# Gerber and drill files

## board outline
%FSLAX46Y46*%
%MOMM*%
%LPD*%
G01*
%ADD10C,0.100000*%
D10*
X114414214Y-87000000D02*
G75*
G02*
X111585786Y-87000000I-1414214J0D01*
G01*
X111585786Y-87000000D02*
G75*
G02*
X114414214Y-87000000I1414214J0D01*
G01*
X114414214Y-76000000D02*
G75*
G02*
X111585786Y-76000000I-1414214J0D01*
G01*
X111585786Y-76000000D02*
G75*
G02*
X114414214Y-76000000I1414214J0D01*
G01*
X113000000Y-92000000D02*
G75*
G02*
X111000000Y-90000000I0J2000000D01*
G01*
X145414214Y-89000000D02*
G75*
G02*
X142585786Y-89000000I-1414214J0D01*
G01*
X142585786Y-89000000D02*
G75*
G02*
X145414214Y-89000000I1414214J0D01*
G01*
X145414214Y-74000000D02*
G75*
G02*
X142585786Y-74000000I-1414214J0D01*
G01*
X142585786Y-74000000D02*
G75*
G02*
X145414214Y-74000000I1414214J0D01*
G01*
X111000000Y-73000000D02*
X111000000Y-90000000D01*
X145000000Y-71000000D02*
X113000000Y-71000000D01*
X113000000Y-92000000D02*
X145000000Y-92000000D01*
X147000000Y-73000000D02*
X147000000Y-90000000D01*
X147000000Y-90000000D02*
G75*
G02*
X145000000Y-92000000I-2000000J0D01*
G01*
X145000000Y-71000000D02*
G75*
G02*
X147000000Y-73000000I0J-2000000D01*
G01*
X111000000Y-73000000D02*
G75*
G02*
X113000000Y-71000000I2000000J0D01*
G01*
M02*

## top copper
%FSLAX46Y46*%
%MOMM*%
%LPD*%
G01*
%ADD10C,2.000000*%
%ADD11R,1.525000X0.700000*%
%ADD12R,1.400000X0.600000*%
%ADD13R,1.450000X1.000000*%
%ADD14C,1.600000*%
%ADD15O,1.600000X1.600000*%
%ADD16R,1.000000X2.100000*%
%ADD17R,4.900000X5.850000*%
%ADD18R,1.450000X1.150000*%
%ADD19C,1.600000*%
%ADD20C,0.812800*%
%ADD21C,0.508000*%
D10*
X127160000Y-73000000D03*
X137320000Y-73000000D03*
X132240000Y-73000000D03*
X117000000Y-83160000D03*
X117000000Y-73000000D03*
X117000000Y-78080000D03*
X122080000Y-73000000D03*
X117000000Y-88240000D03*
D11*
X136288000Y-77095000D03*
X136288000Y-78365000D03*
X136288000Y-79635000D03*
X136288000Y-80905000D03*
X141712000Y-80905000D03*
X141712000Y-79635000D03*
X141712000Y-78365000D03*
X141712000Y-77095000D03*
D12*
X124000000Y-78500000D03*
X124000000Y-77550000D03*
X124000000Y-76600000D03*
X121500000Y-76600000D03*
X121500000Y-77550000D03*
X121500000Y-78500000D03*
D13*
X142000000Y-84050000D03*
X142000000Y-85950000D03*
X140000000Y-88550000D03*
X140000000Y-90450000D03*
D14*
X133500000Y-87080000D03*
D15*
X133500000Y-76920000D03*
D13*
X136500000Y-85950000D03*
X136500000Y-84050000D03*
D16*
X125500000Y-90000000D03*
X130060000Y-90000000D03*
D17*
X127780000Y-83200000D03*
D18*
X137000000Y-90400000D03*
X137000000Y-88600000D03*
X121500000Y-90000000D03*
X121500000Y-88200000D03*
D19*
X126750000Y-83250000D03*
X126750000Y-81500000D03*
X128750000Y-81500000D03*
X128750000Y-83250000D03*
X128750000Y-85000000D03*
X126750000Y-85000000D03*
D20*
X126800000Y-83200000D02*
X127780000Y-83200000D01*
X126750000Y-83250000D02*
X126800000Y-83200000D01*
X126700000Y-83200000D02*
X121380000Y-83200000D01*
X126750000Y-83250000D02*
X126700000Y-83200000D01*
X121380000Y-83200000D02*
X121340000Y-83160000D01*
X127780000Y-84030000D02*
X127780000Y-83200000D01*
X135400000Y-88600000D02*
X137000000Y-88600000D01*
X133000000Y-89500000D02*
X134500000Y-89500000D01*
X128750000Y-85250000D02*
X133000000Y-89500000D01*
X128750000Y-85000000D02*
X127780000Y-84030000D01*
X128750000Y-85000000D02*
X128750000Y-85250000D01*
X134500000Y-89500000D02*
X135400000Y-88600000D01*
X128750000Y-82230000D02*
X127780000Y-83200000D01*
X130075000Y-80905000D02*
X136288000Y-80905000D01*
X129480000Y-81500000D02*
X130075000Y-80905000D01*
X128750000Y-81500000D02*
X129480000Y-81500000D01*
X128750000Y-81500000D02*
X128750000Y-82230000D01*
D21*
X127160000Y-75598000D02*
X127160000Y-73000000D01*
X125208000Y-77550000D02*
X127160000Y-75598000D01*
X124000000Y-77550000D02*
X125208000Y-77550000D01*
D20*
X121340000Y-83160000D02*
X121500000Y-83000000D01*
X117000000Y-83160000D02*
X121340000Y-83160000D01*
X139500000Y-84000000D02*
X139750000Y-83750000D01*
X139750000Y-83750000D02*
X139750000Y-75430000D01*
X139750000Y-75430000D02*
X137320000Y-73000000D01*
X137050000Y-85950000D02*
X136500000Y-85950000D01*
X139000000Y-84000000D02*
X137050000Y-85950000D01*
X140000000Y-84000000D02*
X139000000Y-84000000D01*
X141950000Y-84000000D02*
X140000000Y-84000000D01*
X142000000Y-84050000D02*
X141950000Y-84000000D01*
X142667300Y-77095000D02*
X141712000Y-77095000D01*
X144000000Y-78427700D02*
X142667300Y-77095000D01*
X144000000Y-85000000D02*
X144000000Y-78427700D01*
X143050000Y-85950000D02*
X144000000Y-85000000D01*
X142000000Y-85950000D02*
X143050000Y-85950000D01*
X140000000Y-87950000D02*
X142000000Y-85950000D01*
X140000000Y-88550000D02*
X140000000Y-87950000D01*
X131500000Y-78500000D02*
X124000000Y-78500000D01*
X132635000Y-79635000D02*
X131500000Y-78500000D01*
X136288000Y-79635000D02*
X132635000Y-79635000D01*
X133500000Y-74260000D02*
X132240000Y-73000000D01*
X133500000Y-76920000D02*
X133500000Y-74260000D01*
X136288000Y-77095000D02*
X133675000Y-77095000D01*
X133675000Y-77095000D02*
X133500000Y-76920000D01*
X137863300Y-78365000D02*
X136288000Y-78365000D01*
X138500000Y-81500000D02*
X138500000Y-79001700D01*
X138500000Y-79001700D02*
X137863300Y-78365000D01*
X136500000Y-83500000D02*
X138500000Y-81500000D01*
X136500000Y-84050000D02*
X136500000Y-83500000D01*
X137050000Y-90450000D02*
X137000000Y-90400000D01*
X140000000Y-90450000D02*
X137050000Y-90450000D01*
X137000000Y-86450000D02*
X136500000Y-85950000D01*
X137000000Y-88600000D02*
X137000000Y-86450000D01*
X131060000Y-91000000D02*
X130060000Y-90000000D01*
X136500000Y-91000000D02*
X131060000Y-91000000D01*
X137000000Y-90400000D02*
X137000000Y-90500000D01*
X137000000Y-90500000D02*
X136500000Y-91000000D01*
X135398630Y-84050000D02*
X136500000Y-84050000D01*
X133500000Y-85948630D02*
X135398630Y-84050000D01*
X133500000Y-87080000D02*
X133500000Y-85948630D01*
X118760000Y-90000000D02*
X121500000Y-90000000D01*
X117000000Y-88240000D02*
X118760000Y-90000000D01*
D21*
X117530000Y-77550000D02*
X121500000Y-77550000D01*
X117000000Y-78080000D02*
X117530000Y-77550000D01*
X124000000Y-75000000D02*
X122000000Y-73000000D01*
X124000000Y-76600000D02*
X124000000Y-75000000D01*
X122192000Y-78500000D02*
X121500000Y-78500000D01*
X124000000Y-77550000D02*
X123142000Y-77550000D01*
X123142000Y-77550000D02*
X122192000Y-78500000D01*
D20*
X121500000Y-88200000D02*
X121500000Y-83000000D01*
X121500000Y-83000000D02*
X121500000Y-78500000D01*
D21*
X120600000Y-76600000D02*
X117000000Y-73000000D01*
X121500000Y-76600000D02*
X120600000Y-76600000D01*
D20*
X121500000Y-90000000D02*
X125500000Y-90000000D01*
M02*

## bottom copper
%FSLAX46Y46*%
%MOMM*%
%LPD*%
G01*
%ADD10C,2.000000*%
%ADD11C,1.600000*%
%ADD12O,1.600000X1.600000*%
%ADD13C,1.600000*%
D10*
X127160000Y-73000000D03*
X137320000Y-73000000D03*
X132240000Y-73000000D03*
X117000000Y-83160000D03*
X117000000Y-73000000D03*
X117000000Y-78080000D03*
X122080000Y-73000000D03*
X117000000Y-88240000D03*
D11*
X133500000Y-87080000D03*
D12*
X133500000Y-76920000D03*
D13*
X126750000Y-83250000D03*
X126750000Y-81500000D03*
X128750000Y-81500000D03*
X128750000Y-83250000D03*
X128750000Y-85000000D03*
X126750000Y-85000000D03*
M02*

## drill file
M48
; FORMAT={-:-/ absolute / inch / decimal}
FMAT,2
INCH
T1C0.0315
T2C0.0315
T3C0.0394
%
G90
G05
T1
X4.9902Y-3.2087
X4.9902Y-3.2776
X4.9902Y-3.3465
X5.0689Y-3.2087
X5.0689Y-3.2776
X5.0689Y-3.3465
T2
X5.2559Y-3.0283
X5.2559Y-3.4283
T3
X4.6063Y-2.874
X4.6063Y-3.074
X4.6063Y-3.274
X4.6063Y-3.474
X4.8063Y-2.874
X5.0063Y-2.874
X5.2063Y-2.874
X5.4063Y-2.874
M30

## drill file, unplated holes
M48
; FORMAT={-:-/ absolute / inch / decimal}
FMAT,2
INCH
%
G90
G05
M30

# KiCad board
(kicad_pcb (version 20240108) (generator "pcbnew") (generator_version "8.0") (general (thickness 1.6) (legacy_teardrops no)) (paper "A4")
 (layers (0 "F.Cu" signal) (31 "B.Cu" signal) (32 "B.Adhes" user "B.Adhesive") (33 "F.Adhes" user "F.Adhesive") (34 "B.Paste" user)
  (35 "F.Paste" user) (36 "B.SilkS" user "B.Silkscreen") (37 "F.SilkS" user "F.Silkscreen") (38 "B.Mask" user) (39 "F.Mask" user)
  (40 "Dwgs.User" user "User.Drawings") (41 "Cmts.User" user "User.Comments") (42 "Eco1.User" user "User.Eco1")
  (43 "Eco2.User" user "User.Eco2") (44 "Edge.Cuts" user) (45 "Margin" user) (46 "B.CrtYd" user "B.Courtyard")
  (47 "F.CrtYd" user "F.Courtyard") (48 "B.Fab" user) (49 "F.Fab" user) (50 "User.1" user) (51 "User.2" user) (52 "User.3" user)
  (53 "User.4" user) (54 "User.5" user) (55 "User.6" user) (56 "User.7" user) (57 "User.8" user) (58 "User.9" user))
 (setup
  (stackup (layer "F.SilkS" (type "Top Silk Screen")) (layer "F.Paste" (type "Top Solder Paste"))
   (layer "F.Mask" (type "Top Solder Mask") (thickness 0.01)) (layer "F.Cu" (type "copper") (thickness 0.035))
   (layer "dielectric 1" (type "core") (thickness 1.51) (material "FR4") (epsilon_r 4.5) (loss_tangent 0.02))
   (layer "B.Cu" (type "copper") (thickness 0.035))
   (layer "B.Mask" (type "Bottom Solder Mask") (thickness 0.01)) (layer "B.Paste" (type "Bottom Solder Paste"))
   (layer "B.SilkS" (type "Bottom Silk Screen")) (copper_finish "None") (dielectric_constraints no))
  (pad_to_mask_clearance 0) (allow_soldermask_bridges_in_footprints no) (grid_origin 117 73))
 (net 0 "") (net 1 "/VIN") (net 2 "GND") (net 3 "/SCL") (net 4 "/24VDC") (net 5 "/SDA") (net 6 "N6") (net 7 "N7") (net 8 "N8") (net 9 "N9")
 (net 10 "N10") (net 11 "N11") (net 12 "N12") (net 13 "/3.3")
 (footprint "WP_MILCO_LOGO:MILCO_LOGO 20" (layer "F.Cu") (at 113.5 81.4 90)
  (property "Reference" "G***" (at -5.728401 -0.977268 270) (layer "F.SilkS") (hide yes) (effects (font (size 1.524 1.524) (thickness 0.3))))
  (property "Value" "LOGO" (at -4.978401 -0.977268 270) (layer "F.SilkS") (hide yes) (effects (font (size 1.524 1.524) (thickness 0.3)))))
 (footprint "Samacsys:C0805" (layer "F.Cu") (at 121.5 89.1 90)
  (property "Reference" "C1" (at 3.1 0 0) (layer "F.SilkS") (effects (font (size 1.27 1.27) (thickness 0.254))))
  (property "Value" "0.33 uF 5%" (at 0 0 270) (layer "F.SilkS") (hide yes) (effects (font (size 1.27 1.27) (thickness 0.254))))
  (pad "1" smd rect (at -0.9 0 90) (size 1.15 1.45) (layers "F.Cu" "F.Paste" "F.Mask") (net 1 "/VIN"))
  (pad "2" smd rect (at 0.9 0 90) (size 1.15 1.45) (layers "F.Cu" "F.Paste" "F.Mask") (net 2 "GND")))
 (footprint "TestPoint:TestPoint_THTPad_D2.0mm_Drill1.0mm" (layer "F.Cu") (at 127.16 73)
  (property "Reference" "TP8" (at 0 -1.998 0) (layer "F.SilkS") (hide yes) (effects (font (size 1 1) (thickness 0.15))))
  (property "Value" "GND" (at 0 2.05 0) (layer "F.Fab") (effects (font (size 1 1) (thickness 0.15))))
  (pad "1" thru_hole circle (at 0 0) (size 2 2) (drill 1) (layers "*.Cu" "*.Mask") (remove_unused_layers no) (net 2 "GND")))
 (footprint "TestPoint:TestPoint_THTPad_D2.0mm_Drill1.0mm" (layer "F.Cu") (at 117 78.08)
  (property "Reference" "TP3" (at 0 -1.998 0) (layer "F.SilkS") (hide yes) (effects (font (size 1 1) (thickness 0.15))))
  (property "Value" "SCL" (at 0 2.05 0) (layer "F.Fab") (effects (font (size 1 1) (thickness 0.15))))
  (pad "1" thru_hole circle (at 0 0) (size 2 2) (drill 1) (layers "*.Cu" "*.Mask") (remove_unused_layers no) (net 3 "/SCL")))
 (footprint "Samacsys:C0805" (layer "F.Cu") (at 137 89.5 90)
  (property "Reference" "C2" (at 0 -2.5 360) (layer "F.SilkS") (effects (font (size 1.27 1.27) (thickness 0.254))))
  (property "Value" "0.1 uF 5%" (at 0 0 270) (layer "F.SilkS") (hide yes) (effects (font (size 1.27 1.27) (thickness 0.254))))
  (pad "1" smd rect (at -0.9 0 90) (size 1.15 1.45) (layers "F.Cu" "F.Paste" "F.Mask") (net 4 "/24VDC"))
  (pad "2" smd rect (at 0.9 0 90) (size 1.15 1.45) (layers "F.Cu" "F.Paste" "F.Mask") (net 2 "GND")))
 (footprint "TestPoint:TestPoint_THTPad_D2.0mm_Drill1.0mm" (layer "F.Cu") (at 117 73)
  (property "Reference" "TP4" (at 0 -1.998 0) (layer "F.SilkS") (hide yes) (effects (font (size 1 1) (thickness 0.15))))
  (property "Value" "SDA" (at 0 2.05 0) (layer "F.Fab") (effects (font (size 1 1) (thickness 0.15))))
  (pad "1" thru_hole circle (at 0 0) (size 2 2) (drill 1) (layers "*.Cu" "*.Mask") (remove_unused_layers no) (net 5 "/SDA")))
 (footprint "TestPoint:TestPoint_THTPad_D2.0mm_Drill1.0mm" (layer "F.Cu") (at 117 83.16)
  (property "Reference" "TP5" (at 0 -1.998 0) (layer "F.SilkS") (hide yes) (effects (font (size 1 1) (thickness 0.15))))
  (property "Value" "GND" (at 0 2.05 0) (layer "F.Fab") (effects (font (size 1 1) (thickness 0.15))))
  (pad "1" thru_hole circle (at 0 0) (size 2 2) (drill 1) (layers "*.Cu" "*.Mask") (remove_unused_layers no) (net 2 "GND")))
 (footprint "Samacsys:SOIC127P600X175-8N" (layer "F.Cu") (at 139 79)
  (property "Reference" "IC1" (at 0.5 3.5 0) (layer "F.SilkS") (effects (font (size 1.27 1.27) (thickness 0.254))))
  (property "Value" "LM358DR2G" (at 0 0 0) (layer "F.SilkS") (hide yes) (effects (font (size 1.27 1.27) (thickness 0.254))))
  (pad "1" smd rect (at -2.712 -1.905 90) (size 0.7 1.525) (layers "F.Cu" "F.Paste" "F.Mask") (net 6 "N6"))
  (pad "2" smd rect (at -2.712 -0.635 90) (size 0.7 1.525) (layers "F.Cu" "F.Paste" "F.Mask") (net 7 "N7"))
  (pad "3" smd rect (at -2.712 0.635 90) (size 0.7 1.525) (layers "F.Cu" "F.Paste" "F.Mask") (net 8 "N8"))
  (pad "4" smd rect (at -2.712 1.905 90) (size 0.7 1.525) (layers "F.Cu" "F.Paste" "F.Mask") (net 2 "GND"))
  (pad "5" smd rect (at 2.712 1.905 90) (size 0.7 1.525) (layers "F.Cu" "F.Paste" "F.Mask") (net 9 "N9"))
  (pad "6" smd rect (at 2.712 0.635 90) (size 0.7 1.525) (layers "F.Cu" "F.Paste" "F.Mask") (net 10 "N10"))
  (pad "7" smd rect (at 2.712 -0.635 90) (size 0.7 1.525) (layers "F.Cu" "F.Paste" "F.Mask") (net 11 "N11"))
  (pad "8" smd rect (at 2.712 -1.905 90) (size 0.7 1.525) (layers "F.Cu" "F.Paste" "F.Mask") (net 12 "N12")))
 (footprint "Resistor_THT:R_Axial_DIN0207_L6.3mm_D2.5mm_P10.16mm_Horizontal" (layer "F.Cu") (at 133.5 87.08 90)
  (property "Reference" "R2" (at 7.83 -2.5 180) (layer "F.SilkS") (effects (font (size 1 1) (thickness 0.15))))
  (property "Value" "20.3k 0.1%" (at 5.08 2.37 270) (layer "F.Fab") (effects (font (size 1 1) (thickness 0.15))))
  (pad "1" thru_hole circle (at 0 0 90) (size 1.6 1.6) (drill 0.8) (layers "*.Cu" "*.Mask") (remove_unused_layers no) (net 7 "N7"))
  (pad "2" thru_hole oval (at 10.16 0 90) (size 1.6 1.6) (drill 0.8) (layers "*.Cu" "*.Mask") (remove_unused_layers no) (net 6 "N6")))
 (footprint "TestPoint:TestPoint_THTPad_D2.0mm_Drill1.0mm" (layer "F.Cu") (at 132.24 73)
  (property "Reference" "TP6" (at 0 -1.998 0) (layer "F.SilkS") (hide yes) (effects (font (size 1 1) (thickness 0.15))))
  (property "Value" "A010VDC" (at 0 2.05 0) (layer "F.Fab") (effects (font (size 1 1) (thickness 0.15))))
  (pad "1" thru_hole circle (at 0 0) (size 2 2) (drill 1) (layers "*.Cu" "*.Mask") (remove_unused_layers no) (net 6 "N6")))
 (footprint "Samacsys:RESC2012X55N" (layer "F.Cu") (at 136.5 85 90)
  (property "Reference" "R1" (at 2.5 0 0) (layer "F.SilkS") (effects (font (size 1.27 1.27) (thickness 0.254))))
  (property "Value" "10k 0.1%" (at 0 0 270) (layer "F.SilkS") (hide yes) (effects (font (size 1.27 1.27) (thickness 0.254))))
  (pad "1" smd rect (at -0.95 0 90) (size 1 1.45) (layers "F.Cu" "F.Paste" "F.Mask") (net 2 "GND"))
  (pad "2" smd rect (at 0.95 0 90) (size 1 1.45) (layers "F.Cu" "F.Paste" "F.Mask") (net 7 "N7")))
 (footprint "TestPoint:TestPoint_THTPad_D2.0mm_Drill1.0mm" (layer "F.Cu") (at 137.32 73)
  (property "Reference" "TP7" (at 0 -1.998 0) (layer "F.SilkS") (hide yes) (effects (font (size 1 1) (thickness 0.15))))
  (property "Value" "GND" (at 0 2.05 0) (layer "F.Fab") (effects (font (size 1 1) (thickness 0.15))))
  (pad "1" thru_hole circle (at 0 0) (size 2 2) (drill 1) (layers "*.Cu" "*.Mask") (remove_unused_layers no) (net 2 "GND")))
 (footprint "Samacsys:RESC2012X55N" (layer "F.Cu") (at 140 89.5 -90)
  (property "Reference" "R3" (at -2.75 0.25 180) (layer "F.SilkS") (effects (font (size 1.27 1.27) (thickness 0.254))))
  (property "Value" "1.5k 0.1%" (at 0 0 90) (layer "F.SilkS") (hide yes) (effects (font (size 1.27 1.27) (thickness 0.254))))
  (pad "1" smd rect (at -0.95 0 270) (size 1 1.45) (layers "F.Cu" "F.Paste" "F.Mask") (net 12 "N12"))
  (pad "2" smd rect (at 0.95 0 270) (size 1 1.45) (layers "F.Cu" "F.Paste" "F.Mask") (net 4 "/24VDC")))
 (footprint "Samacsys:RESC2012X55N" (layer "F.Cu") (at 142 85 -90)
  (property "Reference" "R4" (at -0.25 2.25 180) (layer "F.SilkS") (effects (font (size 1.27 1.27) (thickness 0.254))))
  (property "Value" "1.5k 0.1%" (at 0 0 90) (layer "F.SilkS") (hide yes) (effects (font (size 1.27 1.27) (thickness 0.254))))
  (pad "1" smd rect (at -0.95 0 270) (size 1 1.45) (layers "F.Cu" "F.Paste" "F.Mask") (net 2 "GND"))
  (pad "2" smd rect (at 0.95 0 270) (size 1 1.45) (layers "F.Cu" "F.Paste" "F.Mask") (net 12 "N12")))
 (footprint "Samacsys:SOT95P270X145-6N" (layer "F.Cu") (at 122.75 77.55 180)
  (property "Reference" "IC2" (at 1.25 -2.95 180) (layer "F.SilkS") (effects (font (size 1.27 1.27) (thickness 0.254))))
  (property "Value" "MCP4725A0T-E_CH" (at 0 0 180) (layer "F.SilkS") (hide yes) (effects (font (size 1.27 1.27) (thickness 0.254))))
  (pad "1" smd rect (at -1.25 -0.95 270) (size 0.6 1.4) (layers "F.Cu" "F.Paste" "F.Mask") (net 8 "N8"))
  (pad "2" smd rect (at -1.25 0 270) (size 0.6 1.4) (layers "F.Cu" "F.Paste" "F.Mask") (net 2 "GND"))
  (pad "3" smd rect (at -1.25 0.95 270) (size 0.6 1.4) (layers "F.Cu" "F.Paste" "F.Mask") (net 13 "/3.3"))
  (pad "4" smd rect (at 1.25 0.95 270) (size 0.6 1.4) (layers "F.Cu" "F.Paste" "F.Mask") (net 5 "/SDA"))
  (pad "5" smd rect (at 1.25 0 270) (size 0.6 1.4) (layers "F.Cu" "F.Paste" "F.Mask") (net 3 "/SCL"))
  (pad "6" smd rect (at 1.25 -0.95 270) (size 0.6 1.4) (layers "F.Cu" "F.Paste" "F.Mask") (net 2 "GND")))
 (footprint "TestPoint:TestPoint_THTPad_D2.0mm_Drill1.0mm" (layer "F.Cu") (at 117 88.24)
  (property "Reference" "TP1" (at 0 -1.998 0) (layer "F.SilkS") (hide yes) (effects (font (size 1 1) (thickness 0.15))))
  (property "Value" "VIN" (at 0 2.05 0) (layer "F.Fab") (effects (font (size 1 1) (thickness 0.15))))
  (pad "1" thru_hole circle (at 0 0) (size 2 2) (drill 1) (layers "*.Cu" "*.Mask") (remove_unused_layers no) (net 1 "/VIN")))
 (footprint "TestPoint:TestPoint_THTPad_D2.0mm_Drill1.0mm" (layer "F.Cu") (at 122.08 73)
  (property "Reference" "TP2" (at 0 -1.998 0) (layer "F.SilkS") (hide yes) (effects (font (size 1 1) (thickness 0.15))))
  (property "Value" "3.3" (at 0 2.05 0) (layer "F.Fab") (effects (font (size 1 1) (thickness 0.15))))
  (pad "1" thru_hole circle (at 0 0) (size 2 2) (drill 1) (layers "*.Cu" "*.Mask") (remove_unused_layers no) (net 13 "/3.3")))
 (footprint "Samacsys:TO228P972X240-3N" (layer "F.Cu") (at 127.78 85.65 90)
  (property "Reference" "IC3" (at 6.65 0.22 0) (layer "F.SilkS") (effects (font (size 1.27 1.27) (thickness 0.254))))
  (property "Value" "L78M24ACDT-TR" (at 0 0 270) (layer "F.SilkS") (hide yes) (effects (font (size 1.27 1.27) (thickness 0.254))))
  (pad "1" smd rect (at -4.35 -2.28 180) (size 1 2.1) (layers "F.Cu" "F.Paste" "F.Mask") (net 1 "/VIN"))
  (pad "3" smd rect (at -4.35 2.28 180) (size 1 2.1) (layers "F.Cu" "F.Paste" "F.Mask") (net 4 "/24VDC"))
  (pad "4" smd rect (at 2.45 0 180) (size 4.9 5.85) (layers "F.Cu" "F.Paste" "F.Mask") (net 2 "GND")))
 (gr_arc (start 111 73) (mid 111.585786 71.585786) (end 113 71) (stroke (width 0.1) (type default)) (layer "Edge.Cuts"))
 (gr_circle (center 144 89) (end 145 90) (stroke (width 0.1) (type default)) (fill none) (layer "Edge.Cuts"))
 (gr_arc (start 145 71) (mid 146.414214 71.585786) (end 147 73) (stroke (width 0.1) (type default)) (layer "Edge.Cuts"))
 (gr_circle (center 113 87) (end 112 86) (stroke (width 0.1) (type default)) (fill none) (layer "Edge.Cuts"))
 (gr_line (start 145 71) (end 113 71) (stroke (width 0.1) (type default)) (layer "Edge.Cuts"))
 (gr_circle (center 113 76) (end 112 75) (stroke (width 0.1) (type default)) (fill none) (layer "Edge.Cuts"))
 (gr_line (start 147 73) (end 147 90) (stroke (width 0.1) (type default)) (layer "Edge.Cuts"))
 (gr_arc (start 113 92) (mid 111.585786 91.414214) (end 111 90) (stroke (width 0.1) (type default)) (layer "Edge.Cuts"))
 (gr_circle (center 144 74) (end 145 73) (stroke (width 0.1) (type default)) (fill none) (layer "Edge.Cuts"))
 (gr_line (start 113 92) (end 145 92) (stroke (width 0.1) (type default)) (layer "Edge.Cuts"))
 (gr_arc (start 147 90) (mid 146.414214 91.414214) (end 145 92) (stroke (width 0.1) (type default)) (layer "Edge.Cuts"))
 (gr_line (start 111 73) (end 111 90) (stroke (width 0.1) (type default)) (layer "Edge.Cuts"))
 (segment (start 118.76 90) (end 121.5 90) (width 0.8128) (layer "F.Cu") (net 1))
 (segment (start 121.5 90) (end 125.5 90) (width 0.8128) (layer "F.Cu") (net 1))
 (segment (start 117 88.24) (end 118.76 90) (width 0.8128) (layer "F.Cu") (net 1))
 (segment (start 126.75 83.25) (end 126.7 83.2) (width 0.8128) (layer "F.Cu") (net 2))
 (segment (start 117 83.16) (end 121.34 83.16) (width 0.8128) (layer "F.Cu") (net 2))
 (segment (start 139.5 84) (end 139.75 83.75) (width 0.8128) (layer "F.Cu") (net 2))
 (segment (start 128.75 85.25) (end 133 89.5) (width 0.8128) (layer "F.Cu") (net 2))
 (segment (start 139 84) (end 137.05 85.95) (width 0.8128) (layer "F.Cu") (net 2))
 (segment (start 126.8 83.2) (end 127.78 83.2) (width 0.8128) (layer "F.Cu") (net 2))
 (segment (start 142 84.05) (end 141.95 84) (width 0.8128) (layer "F.Cu") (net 2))
 (segment (start 121.38 83.2) (end 121.34 83.16) (width 0.8128) (layer "F.Cu") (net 2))
 (segment (start 121.5 88.2) (end 121.5 83) (width 0.8128) (layer "F.Cu") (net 2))
 (segment (start 123.142 77.55) (end 122.192 78.5) (width 0.508) (layer "F.Cu") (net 2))
 (segment (start 128.75 82.23) (end 127.78 83.2) (width 0.8128) (layer "F.Cu") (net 2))
 (segment (start 121.5 83) (end 121.5 78.5) (width 0.8128) (layer "F.Cu") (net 2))
 (segment (start 126.7 83.2) (end 121.38 83.2) (width 0.8128) (layer "F.Cu") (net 2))
 (segment (start 126.75 83.25) (end 126.8 83.2) (width 0.8128) (layer "F.Cu") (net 2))
 (segment (start 140 84) (end 139 84) (width 0.8128) (layer "F.Cu") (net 2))
 (segment (start 137.05 85.95) (end 136.5 85.95) (width 0.8128) (layer "F.Cu") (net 2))
 (segment (start 137 88.6) (end 137 86.45) (width 0.8128) (layer "F.Cu") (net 2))
 (segment (start 133 89.5) (end 134.5 89.5) (width 0.8128) (layer "F.Cu") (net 2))
 (segment (start 129.48 81.5) (end 130.075 80.905) (width 0.8128) (layer "F.Cu") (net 2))
 (segment (start 124 77.55) (end 123.142 77.55) (width 0.508) (layer "F.Cu") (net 2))
 (segment (start 139.75 83.75) (end 139.75 75.43) (width 0.8128) (layer "F.Cu") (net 2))
 (segment (start 128.75 85) (end 128.75 85.25) (width 0.8128) (layer "F.Cu") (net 2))
 (segment (start 127.16 75.598) (end 127.16 73) (width 0.508) (layer "F.Cu") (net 2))
 (segment (start 141.95 84) (end 140 84) (width 0.8128) (layer "F.Cu") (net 2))
 (segment (start 135.4 88.6) (end 137 88.6) (width 0.8128) (layer "F.Cu") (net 2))
 (segment (start 128.75 81.5) (end 128.75 82.23) (width 0.8128) (layer "F.Cu") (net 2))
 (segment (start 121.34 83.16) (end 121.5 83) (width 0.8128) (layer "F.Cu") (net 2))
 (segment (start 128.75 81.5) (end 129.48 81.5) (width 0.8128) (layer "F.Cu") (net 2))
 (segment (start 137 86.45) (end 136.5 85.95) (width 0.8128) (layer "F.Cu") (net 2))
 (segment (start 122.192 78.5) (end 121.5 78.5) (width 0.508) (layer "F.Cu") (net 2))
 (segment (start 127.78 84.03) (end 127.78 83.2) (width 0.8128) (layer "F.Cu") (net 2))
 (segment (start 130.075 80.905) (end 136.288 80.905) (width 0.8128) (layer "F.Cu") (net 2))
 (segment (start 128.75 85) (end 127.78 84.03) (width 0.8128) (layer "F.Cu") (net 2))
 (segment (start 134.5 89.5) (end 135.4 88.6) (width 0.8128) (layer "F.Cu") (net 2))
 (segment (start 139.75 75.43) (end 137.32 73) (width 0.8128) (layer "F.Cu") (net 2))
 (segment (start 124 77.55) (end 125.208 77.55) (width 0.508) (layer "F.Cu") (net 2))
 (segment (start 125.208 77.55) (end 127.16 75.598) (width 0.508) (layer "F.Cu") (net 2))
 (via (at 128.75 81.5) (size 1.6) (drill 0.8) (layers "F.Cu" "B.Cu") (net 2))
 (via (at 128.75 83.25) (size 1.6) (drill 0.8) (layers "F.Cu" "B.Cu") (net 2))
 (via (at 128.75 85) (size 1.6) (drill 0.8) (layers "F.Cu" "B.Cu") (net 2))
 (via (at 126.75 83.25) (size 1.6) (drill 0.8) (layers "F.Cu" "B.Cu") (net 2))
 (via (at 126.75 85) (size 1.6) (drill 0.8) (layers "F.Cu" "B.Cu") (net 2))
 (via (at 126.75 81.5) (size 1.6) (drill 0.8) (layers "F.Cu" "B.Cu") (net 2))
 (segment (start 137.05 90.45) (end 137 90.4) (width 0.8128) (layer "F.Cu") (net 4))
 (segment (start 137 90.4) (end 137 90.5) (width 0.8128) (layer "F.Cu") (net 4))
 (segment (start 136.5 91) (end 131.06 91) (width 0.8128) (layer "F.Cu") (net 4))
 (segment (start 140 90.45) (end 137.05 90.45) (width 0.8128) (layer "F.Cu") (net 4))
 (segment (start 137 90.5) (end 136.5 91) (width 0.8128) (layer "F.Cu") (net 4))
 (segment (start 131.06 91) (end 130.06 90) (width 0.8128) (layer "F.Cu") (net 4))
 (segment (start 133.675 77.095) (end 133.5 76.92) (width 0.8128) (layer "F.Cu") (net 6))
 (segment (start 133.5 74.26) (end 132.24 73) (width 0.8128) (layer "F.Cu") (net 6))
 (segment (start 136.288 77.095) (end 133.675 77.095) (width 0.8128) (layer "F.Cu") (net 6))
 (segment (start 133.5 76.92) (end 133.5 74.26) (width 0.8128) (layer "F.Cu") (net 6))
 (segment (start 136.5 84.05) (end 136.5 83.5) (width 0.8128) (layer "F.Cu") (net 7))
 (segment (start 136.5 83.5) (end 138.5 81.5) (width 0.8128) (layer "F.Cu") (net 7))
 (segment (start 138.5 79.0017) (end 137.8633 78.365) (width 0.8128) (layer "F.Cu") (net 7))
 (segment (start 137.8633 78.365) (end 136.288 78.365) (width 0.8128) (layer "F.Cu") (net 7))
 (segment (start 138.5 81.5) (end 138.5 79.0017) (width 0.8128) (layer "F.Cu") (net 7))
 (segment (start 133.5 87.08) (end 133.5 85.94863) (width 0.8128) (layer "F.Cu") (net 7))
 (segment (start 135.39863 84.05) (end 136.5 84.05) (width 0.8128) (layer "F.Cu") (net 7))
 (segment (start 133.5 85.94863) (end 135.39863 84.05) (width 0.8128) (layer "F.Cu") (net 7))
 (segment (start 132.635 79.635) (end 131.5 78.5) (width 0.8128) (layer "F.Cu") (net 8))
 (segment (start 131.5 78.5) (end 124 78.5) (width 0.8128) (layer "F.Cu") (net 8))
 (segment (start 136.288 79.635) (end 132.635 79.635) (width 0.8128) (layer "F.Cu") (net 8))
 (segment (start 144 85) (end 144 78.4277) (width 0.8128) (layer "F.Cu") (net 12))
 (segment (start 142.6673 77.095) (end 141.712 77.095) (width 0.8128) (layer "F.Cu") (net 12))
 (segment (start 140 88.55) (end 140 87.95) (width 0.8128) (layer "F.Cu") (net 12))
 (segment (start 144 78.4277) (end 142.6673 77.095) (width 0.8128) (layer "F.Cu") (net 12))
 (segment (start 142 85.95) (end 143.05 85.95) (width 0.8128) (layer "F.Cu") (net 12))
 (segment (start 143.05 85.95) (end 144 85) (width 0.8128) (layer "F.Cu") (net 12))
 (segment (start 140 87.95) (end 142 85.95) (width 0.8128) (layer "F.Cu") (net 12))
 (segment (start 120.6 76.6) (end 117 73) (width 0.508) (layer "F.Cu") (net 5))
 (segment (start 121.5 76.6) (end 120.6 76.6) (width 0.508) (layer "F.Cu") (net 5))
 (segment (start 117.53 77.55) (end 121.5 77.55) (width 0.508) (layer "F.Cu") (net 3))
 (segment (start 117 78.08) (end 117.53 77.55) (width 0.508) (layer "F.Cu") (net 3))
 (segment (start 124 76.6) (end 124 75) (width 0.508) (layer "F.Cu") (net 13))
 (segment (start 124 75) (end 122 73) (width 0.508) (layer "F.Cu") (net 13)))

